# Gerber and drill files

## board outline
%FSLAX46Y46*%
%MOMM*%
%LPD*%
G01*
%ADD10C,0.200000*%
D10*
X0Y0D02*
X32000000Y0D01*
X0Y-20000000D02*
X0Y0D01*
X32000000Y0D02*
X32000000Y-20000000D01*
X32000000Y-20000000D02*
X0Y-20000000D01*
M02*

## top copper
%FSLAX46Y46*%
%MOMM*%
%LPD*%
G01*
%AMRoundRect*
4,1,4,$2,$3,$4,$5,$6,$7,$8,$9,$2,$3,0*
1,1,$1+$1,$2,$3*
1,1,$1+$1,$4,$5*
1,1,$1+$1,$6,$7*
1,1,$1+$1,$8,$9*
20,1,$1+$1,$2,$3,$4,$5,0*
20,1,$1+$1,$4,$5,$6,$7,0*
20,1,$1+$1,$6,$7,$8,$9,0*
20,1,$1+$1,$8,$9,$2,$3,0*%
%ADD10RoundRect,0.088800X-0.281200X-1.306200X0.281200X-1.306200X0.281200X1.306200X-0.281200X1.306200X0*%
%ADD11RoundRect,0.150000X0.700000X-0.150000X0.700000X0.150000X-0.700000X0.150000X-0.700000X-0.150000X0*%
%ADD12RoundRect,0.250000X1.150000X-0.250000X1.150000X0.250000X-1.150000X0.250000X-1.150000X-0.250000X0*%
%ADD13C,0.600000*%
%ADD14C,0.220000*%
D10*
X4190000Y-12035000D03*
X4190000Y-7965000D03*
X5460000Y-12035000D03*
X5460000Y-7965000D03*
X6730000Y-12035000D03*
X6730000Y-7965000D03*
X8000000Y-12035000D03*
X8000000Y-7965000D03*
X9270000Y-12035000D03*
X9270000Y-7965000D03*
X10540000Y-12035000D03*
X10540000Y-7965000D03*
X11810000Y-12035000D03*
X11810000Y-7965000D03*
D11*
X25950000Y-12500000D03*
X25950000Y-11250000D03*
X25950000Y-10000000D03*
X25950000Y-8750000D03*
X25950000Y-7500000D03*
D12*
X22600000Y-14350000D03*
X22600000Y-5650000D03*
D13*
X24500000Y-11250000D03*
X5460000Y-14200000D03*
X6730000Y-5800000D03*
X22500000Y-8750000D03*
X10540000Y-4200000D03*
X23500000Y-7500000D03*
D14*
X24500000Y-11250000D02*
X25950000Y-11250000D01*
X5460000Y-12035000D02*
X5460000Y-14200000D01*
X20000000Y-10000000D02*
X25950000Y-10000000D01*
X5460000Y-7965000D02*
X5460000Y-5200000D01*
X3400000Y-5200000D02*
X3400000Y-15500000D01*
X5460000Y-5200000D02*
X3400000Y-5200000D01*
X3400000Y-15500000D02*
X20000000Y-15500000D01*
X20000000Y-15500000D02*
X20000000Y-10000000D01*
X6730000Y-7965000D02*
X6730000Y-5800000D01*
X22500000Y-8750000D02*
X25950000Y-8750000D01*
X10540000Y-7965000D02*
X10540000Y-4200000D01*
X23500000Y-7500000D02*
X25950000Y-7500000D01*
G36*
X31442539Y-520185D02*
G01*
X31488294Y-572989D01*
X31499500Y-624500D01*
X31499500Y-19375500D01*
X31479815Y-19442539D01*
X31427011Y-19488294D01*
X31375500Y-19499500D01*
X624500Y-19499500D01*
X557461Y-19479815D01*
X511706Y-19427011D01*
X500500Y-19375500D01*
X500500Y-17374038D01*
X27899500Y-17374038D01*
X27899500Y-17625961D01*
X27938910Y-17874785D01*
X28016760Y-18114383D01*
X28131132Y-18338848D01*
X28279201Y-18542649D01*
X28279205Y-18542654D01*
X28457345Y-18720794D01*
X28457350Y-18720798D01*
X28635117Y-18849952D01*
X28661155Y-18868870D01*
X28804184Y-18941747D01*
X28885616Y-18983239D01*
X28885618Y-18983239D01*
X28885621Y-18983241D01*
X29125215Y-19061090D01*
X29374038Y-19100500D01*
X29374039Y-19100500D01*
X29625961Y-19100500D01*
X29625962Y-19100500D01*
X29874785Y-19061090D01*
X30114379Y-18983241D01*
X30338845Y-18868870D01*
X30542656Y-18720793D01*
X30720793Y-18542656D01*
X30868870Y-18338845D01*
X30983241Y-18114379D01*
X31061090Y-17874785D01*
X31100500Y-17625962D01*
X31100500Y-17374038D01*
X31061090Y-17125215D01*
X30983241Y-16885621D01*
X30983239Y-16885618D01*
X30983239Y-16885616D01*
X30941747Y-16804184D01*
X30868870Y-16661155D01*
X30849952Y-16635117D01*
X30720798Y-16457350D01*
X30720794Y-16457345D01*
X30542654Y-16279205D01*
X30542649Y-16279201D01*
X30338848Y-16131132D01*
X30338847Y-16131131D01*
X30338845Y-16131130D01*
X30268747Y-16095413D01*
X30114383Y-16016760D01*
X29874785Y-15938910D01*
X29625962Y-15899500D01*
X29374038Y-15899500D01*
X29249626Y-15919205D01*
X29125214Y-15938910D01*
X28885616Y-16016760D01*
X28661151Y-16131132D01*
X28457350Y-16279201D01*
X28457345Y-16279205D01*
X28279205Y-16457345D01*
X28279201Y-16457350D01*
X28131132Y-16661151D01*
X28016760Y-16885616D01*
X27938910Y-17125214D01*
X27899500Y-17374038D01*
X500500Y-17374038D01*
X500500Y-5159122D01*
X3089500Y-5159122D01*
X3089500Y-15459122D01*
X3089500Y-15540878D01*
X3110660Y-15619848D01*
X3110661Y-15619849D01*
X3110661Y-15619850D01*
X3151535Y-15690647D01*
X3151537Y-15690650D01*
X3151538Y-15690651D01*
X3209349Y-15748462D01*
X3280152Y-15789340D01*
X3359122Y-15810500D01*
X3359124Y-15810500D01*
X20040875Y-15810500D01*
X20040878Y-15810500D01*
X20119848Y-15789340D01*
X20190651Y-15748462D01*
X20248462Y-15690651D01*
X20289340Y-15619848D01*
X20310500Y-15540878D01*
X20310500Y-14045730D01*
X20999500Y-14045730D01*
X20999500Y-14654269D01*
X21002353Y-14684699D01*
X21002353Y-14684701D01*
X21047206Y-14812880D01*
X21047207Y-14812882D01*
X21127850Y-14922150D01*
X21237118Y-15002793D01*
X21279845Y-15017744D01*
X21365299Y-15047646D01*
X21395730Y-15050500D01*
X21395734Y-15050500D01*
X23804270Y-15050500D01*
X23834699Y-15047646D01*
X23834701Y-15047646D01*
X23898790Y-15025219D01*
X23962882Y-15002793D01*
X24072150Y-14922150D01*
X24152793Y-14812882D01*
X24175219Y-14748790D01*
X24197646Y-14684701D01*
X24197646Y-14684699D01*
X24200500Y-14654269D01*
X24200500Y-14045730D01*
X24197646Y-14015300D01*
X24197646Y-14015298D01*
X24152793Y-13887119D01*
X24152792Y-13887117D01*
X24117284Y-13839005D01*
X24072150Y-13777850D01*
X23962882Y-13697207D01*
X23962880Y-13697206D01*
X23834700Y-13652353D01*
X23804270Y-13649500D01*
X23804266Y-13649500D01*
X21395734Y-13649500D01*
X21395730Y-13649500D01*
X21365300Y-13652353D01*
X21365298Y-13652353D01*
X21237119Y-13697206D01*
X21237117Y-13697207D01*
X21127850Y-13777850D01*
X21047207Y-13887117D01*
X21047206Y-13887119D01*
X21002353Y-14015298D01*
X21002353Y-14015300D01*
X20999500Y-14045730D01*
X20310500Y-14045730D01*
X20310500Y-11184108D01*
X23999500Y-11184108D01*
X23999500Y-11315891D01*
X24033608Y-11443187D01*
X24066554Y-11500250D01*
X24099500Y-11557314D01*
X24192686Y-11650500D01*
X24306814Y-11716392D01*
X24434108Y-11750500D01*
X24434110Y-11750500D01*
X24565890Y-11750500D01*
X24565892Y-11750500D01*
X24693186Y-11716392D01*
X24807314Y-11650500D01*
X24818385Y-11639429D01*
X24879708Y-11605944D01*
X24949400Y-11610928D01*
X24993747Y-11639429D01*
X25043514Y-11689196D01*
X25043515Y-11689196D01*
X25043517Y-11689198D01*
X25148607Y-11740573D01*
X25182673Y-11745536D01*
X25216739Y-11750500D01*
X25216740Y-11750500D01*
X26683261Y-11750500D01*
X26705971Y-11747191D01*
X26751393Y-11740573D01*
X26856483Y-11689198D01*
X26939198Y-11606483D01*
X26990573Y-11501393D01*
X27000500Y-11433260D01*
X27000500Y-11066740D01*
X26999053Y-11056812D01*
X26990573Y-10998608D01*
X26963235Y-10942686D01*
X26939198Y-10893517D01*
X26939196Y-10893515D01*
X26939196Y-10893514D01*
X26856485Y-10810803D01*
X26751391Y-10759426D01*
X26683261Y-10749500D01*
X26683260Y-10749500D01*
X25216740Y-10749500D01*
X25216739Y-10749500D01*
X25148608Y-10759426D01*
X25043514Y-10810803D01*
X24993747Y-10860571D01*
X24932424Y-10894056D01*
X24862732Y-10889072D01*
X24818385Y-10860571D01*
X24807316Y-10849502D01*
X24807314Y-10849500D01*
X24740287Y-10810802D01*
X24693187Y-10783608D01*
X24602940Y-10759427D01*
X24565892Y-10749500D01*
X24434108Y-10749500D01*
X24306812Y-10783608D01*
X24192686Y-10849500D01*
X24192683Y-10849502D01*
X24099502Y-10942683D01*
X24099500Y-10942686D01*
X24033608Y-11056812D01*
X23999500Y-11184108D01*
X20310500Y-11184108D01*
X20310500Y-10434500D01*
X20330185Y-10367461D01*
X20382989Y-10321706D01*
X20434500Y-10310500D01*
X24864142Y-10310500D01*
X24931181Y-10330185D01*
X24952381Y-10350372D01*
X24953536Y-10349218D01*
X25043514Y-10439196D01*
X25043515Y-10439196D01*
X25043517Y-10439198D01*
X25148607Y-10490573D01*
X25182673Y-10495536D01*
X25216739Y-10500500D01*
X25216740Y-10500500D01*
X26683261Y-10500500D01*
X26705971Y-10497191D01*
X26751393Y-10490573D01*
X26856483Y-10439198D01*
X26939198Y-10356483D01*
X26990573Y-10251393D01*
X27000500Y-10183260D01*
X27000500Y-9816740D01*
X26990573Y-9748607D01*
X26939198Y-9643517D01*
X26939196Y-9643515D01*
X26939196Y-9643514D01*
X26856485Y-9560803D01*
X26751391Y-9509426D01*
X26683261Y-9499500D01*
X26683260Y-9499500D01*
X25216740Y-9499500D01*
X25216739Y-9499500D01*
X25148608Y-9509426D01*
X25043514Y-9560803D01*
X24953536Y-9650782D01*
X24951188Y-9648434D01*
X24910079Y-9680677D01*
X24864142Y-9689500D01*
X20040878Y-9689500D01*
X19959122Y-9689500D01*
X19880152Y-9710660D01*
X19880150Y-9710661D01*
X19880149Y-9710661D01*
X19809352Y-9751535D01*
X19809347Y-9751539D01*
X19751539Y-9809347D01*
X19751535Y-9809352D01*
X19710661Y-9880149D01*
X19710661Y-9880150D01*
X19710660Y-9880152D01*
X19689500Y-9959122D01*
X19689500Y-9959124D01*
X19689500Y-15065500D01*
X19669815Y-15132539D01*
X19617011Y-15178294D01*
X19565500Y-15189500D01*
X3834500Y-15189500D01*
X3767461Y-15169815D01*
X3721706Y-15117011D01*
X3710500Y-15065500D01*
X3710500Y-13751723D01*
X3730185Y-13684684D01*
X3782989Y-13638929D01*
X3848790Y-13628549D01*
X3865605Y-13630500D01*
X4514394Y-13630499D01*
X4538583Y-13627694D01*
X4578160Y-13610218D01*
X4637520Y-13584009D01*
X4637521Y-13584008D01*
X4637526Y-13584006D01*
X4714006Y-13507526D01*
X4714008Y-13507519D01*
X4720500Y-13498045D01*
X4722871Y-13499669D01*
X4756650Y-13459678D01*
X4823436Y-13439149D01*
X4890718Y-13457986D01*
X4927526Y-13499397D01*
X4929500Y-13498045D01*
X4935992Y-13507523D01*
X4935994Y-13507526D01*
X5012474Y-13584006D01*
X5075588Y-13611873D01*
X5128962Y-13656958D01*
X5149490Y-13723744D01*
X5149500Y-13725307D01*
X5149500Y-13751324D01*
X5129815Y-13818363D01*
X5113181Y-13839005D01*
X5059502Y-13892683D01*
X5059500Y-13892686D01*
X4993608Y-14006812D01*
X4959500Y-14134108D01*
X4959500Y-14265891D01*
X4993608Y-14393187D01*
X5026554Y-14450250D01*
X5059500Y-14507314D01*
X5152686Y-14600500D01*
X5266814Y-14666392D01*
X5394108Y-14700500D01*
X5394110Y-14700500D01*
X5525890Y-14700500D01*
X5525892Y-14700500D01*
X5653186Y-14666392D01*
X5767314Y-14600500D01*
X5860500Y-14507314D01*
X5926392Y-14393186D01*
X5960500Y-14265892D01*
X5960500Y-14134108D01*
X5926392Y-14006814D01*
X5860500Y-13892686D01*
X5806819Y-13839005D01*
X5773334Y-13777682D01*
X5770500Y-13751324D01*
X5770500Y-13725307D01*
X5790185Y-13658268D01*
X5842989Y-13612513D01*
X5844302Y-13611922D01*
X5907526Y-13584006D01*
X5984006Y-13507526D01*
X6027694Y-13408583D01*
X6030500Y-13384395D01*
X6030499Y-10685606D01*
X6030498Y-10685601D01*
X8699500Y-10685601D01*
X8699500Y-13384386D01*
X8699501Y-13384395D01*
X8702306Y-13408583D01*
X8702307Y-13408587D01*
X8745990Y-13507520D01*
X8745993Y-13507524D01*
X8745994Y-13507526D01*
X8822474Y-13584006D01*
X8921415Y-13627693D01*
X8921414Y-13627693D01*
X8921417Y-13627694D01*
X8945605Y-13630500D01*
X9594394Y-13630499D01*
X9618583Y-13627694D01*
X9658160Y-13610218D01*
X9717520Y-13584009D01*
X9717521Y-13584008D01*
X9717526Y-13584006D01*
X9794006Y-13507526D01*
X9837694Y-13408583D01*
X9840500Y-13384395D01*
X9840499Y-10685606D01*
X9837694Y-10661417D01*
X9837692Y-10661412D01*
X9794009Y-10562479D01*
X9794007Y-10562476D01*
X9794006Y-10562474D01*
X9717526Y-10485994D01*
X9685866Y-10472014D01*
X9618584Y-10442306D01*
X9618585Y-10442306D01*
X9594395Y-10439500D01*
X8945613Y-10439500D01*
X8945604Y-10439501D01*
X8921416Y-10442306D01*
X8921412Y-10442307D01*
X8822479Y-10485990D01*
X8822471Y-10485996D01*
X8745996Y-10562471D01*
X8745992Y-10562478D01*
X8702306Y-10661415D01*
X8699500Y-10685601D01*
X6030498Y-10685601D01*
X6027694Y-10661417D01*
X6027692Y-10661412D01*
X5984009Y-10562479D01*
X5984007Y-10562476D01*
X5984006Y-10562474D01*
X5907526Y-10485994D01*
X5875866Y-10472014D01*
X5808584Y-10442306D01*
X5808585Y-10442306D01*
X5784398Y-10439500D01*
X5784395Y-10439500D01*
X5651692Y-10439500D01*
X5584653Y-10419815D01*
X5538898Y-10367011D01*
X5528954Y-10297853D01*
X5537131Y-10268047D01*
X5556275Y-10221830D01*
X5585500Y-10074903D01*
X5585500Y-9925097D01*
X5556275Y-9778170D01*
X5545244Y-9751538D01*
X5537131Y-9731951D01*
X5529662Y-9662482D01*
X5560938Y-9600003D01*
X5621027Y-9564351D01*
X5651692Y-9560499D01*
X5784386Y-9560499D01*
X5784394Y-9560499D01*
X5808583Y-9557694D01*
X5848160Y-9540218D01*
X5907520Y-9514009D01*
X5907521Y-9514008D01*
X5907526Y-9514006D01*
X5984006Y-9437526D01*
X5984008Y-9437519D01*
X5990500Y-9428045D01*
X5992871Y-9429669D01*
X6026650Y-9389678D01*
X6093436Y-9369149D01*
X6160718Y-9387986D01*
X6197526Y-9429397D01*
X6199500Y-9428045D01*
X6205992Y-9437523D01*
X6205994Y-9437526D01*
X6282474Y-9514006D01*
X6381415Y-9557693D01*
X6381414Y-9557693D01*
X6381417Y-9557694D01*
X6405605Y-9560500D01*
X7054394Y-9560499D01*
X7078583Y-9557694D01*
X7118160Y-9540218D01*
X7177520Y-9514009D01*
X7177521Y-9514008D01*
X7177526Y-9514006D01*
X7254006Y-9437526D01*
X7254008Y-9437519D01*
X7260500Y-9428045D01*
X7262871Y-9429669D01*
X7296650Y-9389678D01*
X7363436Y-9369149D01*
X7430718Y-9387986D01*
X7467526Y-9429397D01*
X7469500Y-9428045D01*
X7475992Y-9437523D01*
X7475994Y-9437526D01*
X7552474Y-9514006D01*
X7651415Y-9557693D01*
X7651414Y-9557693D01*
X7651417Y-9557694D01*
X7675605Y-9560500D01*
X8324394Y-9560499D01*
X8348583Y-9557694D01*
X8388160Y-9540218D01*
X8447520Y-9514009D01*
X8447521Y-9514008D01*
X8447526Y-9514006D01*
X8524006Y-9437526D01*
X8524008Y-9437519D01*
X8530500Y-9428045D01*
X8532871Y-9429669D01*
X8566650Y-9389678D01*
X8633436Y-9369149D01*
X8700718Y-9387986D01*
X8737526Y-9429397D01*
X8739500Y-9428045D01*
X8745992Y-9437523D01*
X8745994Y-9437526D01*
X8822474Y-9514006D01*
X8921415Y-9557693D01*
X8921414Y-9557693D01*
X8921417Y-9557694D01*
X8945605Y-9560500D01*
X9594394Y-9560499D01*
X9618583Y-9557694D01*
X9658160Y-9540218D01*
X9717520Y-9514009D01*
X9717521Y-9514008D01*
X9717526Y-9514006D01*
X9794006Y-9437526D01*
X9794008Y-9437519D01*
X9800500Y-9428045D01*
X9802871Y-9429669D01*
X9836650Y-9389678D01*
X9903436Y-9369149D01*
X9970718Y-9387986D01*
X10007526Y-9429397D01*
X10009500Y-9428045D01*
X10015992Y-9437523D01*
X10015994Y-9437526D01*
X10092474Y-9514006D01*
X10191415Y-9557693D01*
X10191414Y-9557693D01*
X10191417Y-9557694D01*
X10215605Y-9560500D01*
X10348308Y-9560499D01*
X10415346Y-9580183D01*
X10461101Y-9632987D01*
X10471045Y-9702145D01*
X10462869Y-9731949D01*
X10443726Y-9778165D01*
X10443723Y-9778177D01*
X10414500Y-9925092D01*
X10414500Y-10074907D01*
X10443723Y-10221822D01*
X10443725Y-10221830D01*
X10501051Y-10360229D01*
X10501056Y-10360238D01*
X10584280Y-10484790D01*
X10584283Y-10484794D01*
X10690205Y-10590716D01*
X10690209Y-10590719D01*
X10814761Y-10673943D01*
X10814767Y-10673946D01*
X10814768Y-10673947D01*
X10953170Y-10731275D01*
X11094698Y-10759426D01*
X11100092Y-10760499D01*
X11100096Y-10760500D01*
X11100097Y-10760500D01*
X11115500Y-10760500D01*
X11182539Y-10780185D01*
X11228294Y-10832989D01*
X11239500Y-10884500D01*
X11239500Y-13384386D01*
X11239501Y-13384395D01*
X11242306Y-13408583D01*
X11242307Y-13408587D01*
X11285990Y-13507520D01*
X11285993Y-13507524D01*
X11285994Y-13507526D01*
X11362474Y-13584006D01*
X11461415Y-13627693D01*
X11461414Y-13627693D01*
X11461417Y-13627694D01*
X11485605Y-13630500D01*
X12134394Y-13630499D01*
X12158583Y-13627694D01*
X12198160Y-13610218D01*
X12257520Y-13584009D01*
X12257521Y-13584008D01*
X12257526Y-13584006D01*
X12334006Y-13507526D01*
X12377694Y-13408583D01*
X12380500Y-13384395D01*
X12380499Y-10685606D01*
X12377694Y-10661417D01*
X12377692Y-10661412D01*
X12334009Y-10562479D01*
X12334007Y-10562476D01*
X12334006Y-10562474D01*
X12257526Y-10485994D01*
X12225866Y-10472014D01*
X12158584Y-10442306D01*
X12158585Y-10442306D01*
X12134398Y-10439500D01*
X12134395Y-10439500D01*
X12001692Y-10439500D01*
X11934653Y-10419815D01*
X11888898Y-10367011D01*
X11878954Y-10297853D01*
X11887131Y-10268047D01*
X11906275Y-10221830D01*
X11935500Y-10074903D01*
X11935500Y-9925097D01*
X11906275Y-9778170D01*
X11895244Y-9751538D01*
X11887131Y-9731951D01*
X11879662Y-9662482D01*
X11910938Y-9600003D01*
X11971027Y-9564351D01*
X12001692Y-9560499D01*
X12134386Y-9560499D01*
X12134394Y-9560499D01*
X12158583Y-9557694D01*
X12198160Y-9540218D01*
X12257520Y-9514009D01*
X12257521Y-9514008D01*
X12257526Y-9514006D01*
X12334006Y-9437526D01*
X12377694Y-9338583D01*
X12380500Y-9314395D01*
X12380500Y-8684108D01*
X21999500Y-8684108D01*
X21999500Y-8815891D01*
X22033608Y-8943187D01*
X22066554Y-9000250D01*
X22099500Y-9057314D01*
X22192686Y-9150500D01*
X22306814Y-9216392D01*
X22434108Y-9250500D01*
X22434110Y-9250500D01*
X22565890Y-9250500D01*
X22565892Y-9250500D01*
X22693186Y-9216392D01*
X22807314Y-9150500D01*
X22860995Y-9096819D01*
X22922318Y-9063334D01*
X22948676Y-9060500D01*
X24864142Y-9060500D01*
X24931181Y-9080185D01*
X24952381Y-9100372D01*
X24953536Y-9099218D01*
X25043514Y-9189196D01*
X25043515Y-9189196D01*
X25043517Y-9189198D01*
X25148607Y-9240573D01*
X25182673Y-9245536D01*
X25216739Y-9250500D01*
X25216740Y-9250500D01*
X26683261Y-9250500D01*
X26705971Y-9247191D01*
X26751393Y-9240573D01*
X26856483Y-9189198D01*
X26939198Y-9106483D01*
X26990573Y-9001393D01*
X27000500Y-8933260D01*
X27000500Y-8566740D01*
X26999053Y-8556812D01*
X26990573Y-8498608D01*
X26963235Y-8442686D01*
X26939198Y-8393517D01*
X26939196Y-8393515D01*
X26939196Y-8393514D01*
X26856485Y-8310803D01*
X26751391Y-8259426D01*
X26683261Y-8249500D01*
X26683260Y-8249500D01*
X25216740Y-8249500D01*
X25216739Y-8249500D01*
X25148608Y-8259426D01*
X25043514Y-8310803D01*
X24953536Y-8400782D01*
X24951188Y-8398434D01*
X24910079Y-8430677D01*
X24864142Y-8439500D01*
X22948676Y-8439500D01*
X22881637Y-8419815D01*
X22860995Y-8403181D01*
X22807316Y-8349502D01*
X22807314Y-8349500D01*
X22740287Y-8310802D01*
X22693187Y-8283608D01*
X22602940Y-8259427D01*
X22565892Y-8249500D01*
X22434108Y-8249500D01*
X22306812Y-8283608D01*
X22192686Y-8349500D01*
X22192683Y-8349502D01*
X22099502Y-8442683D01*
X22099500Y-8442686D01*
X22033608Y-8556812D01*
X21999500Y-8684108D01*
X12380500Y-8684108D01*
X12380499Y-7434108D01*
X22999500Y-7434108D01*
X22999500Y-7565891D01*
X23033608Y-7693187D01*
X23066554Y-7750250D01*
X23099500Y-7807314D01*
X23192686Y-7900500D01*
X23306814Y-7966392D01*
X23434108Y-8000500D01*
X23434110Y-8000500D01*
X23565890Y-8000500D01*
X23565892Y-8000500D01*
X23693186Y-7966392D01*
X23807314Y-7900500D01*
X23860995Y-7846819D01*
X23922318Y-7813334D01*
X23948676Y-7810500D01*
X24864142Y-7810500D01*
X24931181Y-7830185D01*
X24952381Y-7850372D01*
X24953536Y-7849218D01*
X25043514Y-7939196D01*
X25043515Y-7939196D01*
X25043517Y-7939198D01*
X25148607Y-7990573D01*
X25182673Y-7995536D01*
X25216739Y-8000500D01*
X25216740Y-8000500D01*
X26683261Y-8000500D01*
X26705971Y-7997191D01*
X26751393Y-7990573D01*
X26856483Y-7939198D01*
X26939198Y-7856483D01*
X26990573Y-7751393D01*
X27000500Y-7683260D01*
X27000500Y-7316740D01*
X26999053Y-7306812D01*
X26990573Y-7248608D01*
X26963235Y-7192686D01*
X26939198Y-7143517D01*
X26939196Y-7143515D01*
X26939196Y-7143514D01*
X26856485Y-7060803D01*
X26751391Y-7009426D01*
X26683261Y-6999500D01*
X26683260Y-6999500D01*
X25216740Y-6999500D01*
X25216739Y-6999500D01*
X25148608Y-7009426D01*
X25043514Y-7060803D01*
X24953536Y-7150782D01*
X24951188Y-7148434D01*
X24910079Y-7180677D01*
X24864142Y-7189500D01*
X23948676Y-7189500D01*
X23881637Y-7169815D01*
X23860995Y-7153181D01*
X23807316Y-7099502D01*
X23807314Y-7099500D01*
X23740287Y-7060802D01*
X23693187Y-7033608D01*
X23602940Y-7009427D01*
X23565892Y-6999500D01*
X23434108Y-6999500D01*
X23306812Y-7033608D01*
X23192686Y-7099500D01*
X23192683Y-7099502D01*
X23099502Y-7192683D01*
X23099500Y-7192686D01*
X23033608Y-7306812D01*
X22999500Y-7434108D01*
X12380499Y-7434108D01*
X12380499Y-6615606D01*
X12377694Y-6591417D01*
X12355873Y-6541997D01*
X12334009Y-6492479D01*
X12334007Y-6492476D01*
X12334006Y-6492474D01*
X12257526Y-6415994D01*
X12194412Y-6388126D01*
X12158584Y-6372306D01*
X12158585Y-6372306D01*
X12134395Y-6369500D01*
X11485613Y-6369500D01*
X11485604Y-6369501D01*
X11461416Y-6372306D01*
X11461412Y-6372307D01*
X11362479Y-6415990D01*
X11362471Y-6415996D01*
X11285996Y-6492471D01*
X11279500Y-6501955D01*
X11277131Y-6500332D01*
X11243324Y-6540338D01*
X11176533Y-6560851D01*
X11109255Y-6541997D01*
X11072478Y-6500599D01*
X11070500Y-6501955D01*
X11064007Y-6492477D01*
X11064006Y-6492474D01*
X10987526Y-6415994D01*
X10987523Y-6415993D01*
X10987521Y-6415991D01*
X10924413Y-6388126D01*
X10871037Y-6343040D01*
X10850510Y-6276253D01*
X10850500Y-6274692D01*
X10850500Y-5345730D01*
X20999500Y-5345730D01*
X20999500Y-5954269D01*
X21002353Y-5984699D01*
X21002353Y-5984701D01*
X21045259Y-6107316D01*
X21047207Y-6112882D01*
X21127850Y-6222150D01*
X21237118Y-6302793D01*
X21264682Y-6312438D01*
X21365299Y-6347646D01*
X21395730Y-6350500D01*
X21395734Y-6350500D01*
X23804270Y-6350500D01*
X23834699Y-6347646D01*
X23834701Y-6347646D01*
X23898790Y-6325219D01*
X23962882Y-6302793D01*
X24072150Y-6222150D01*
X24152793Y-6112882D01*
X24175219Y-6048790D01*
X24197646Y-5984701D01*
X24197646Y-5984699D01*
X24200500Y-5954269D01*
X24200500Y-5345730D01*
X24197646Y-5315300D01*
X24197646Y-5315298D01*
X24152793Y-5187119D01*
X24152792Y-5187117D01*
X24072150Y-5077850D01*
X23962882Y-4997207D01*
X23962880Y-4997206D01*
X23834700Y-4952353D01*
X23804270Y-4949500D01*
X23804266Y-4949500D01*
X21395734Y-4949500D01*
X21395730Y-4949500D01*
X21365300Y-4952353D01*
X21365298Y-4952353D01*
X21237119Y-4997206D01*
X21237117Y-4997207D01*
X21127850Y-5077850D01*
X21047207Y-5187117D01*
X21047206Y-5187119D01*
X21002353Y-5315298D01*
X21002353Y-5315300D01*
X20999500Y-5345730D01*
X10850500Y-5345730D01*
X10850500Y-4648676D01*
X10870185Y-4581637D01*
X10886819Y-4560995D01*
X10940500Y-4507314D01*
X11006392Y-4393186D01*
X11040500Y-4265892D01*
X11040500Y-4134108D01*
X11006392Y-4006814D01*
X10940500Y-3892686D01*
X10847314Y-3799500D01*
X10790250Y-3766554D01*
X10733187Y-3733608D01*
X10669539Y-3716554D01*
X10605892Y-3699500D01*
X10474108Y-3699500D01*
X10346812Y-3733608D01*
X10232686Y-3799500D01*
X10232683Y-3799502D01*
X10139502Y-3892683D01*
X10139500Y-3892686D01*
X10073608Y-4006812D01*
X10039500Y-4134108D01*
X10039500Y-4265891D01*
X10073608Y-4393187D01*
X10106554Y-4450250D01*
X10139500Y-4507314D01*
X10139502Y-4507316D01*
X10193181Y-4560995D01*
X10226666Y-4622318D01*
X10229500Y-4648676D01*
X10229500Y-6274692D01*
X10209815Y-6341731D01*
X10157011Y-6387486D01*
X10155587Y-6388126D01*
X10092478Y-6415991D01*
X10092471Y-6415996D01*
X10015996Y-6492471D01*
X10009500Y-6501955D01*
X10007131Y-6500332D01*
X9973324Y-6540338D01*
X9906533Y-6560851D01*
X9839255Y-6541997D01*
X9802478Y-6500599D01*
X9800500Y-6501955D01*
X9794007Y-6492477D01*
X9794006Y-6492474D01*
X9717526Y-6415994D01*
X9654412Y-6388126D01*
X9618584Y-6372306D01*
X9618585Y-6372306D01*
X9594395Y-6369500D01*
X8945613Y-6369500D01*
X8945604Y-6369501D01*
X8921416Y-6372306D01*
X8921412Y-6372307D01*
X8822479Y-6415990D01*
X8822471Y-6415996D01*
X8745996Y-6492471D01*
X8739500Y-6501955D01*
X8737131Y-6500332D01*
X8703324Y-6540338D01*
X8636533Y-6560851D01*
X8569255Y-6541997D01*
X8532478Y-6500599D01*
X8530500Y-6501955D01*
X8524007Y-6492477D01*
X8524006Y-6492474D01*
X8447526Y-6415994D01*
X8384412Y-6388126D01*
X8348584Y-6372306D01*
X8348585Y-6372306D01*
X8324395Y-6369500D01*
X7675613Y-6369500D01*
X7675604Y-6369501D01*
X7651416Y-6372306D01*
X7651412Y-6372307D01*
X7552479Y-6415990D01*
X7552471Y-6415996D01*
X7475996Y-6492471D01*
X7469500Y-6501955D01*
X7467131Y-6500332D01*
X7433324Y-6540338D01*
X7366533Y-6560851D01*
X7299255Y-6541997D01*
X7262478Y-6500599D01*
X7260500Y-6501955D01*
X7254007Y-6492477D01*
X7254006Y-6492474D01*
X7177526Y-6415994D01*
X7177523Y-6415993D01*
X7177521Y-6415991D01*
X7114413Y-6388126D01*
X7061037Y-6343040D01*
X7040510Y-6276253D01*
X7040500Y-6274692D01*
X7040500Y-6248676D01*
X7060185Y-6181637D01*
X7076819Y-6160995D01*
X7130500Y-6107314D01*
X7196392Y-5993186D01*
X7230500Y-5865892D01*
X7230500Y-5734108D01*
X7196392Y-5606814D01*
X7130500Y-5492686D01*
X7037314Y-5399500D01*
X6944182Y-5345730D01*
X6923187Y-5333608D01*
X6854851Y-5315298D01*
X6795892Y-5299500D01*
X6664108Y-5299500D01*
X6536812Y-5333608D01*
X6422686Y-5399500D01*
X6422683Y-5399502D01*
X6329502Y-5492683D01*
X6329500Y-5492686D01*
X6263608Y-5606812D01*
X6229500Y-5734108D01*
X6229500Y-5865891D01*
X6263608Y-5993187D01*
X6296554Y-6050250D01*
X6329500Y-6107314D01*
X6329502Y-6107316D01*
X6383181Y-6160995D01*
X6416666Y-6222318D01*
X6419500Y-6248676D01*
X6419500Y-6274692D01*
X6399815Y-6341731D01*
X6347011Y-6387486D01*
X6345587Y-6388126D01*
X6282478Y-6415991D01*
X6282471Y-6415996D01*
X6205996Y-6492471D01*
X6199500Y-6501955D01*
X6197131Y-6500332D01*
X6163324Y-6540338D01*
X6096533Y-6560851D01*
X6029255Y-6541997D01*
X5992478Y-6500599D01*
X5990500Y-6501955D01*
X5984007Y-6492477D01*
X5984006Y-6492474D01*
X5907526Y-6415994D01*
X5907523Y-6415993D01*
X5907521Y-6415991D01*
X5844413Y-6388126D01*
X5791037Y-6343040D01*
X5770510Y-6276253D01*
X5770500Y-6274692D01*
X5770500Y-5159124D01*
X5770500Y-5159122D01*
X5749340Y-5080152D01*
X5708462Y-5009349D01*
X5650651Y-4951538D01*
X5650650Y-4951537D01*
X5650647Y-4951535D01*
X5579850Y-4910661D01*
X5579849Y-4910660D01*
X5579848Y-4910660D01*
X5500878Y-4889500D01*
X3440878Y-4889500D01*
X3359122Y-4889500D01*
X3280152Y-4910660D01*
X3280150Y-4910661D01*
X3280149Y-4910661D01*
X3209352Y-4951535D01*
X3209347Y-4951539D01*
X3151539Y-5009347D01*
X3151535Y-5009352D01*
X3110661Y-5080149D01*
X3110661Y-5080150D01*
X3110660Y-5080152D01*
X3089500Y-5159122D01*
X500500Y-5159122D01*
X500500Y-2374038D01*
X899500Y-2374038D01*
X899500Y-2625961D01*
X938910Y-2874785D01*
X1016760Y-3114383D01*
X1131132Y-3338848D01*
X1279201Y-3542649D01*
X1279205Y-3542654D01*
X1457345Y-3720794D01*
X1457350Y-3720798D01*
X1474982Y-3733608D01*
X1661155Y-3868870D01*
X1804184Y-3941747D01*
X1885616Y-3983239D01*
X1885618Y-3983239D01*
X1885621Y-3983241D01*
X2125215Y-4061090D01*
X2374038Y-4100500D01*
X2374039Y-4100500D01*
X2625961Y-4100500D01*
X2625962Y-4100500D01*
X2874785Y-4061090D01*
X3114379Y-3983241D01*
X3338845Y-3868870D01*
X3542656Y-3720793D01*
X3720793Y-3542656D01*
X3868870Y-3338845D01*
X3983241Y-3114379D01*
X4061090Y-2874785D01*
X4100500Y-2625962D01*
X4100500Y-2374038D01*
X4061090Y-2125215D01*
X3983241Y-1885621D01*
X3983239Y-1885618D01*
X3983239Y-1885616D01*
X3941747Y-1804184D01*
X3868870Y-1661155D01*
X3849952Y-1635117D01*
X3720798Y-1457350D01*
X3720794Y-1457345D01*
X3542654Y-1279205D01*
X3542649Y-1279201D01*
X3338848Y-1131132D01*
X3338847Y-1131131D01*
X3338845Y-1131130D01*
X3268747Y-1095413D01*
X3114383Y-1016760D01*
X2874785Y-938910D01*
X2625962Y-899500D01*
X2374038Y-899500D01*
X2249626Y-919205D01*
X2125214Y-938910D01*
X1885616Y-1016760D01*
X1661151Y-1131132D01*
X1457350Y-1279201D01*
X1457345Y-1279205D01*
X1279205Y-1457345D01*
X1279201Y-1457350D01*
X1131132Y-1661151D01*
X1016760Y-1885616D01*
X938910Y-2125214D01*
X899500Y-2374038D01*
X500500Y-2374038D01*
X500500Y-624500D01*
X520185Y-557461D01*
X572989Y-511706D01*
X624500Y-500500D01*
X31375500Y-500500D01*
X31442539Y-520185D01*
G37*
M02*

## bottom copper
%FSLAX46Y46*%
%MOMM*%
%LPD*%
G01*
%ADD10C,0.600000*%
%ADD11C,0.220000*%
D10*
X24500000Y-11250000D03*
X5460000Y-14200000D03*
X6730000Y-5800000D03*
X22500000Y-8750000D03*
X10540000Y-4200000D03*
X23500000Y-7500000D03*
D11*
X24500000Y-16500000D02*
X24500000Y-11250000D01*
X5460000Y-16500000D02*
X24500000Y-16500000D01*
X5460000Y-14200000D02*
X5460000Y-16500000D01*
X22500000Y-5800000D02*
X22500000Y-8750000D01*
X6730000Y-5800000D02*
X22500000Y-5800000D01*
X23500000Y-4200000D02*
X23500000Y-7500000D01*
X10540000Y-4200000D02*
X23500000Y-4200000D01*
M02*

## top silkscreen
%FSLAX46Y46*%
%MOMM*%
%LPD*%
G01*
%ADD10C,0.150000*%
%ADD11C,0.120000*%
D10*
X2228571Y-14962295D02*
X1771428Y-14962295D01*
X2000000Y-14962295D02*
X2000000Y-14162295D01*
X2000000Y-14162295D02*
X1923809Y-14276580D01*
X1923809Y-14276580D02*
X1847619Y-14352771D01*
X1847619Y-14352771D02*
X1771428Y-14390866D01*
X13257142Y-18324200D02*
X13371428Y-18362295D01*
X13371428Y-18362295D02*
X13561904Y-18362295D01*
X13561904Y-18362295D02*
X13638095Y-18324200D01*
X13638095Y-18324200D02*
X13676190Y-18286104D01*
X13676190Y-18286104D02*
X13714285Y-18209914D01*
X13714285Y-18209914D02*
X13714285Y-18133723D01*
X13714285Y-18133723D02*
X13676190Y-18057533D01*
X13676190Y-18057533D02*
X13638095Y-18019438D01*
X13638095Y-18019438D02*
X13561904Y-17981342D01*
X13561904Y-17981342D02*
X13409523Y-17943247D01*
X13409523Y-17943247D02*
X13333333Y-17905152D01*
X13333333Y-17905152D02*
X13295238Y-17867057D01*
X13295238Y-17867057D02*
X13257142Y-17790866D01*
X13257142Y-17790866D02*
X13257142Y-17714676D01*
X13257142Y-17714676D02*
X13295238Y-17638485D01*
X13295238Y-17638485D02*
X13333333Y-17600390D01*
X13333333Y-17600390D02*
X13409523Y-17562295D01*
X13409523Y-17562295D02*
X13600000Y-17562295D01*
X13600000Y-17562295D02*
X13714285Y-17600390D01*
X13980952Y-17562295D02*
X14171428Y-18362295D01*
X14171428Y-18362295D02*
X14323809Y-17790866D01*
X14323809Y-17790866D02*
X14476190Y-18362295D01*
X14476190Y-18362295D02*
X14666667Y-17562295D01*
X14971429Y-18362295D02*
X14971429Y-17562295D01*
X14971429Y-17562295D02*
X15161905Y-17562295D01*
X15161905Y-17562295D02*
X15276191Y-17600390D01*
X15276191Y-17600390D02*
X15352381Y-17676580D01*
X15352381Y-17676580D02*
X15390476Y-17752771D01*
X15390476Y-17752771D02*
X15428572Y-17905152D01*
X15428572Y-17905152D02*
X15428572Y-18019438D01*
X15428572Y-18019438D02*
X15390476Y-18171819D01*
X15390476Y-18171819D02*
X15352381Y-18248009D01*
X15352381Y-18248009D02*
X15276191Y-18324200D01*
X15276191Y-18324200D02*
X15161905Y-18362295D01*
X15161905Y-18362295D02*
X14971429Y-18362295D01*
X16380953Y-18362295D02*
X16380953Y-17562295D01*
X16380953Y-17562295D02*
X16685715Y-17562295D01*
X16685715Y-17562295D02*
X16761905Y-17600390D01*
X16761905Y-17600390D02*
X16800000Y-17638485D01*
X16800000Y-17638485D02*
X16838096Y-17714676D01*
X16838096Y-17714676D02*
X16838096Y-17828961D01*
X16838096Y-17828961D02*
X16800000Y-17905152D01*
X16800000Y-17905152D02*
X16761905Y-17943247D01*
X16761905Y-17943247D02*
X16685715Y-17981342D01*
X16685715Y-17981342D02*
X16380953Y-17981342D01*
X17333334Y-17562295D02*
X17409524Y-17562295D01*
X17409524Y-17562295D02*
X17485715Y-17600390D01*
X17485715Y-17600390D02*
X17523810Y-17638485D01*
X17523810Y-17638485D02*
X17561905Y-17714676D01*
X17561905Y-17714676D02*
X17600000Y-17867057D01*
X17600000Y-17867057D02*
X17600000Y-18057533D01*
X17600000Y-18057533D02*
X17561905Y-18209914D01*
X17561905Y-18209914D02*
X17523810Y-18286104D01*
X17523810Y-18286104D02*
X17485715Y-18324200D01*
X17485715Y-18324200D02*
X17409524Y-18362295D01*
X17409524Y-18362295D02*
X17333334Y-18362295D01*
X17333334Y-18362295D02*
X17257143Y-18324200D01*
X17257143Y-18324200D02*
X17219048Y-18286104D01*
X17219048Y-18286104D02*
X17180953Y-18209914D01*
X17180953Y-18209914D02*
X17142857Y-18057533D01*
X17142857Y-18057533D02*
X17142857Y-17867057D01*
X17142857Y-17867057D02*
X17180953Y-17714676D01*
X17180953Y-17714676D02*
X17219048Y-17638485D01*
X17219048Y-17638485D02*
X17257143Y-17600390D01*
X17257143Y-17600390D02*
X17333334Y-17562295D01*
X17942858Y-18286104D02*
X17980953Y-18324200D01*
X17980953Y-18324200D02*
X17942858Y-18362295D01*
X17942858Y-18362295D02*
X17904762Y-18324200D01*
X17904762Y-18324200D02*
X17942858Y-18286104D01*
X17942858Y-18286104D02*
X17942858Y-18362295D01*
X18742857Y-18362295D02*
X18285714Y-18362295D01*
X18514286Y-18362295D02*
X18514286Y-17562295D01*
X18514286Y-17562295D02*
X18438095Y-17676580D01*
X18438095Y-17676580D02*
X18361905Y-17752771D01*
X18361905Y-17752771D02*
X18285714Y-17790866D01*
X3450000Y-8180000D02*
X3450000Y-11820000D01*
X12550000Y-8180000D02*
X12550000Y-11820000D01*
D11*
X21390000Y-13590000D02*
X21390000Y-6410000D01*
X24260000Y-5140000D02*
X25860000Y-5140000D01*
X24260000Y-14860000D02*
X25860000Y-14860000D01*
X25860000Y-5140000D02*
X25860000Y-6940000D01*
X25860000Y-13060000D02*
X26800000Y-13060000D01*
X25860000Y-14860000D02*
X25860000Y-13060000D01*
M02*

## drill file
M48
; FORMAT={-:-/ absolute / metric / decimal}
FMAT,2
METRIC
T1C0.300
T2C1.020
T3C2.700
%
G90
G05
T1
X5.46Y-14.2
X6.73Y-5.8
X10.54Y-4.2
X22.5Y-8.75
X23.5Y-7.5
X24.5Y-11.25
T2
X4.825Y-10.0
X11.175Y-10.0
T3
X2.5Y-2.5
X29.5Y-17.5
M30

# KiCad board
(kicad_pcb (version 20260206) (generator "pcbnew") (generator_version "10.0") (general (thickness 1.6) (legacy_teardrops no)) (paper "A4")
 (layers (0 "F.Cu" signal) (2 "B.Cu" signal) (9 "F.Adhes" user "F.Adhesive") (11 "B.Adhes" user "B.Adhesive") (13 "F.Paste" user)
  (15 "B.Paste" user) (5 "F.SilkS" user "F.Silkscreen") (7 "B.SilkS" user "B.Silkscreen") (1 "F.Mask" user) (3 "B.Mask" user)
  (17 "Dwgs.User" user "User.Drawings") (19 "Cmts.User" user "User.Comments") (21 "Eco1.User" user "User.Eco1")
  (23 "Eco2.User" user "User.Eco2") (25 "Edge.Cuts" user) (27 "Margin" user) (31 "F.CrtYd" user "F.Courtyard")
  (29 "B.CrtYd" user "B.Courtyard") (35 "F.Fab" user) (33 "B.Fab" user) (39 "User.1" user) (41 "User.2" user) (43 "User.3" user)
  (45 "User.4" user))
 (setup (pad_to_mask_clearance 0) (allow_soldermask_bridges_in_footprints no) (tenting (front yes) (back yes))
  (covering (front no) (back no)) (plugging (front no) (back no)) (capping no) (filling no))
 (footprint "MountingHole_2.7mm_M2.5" (layer "F.Cu") (at 2.5 2.5)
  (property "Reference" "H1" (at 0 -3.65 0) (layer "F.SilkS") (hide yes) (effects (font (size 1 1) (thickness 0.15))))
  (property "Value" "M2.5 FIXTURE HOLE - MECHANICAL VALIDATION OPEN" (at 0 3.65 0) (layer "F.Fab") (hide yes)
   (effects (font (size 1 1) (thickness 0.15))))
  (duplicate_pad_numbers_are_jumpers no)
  (pad "" np_thru_hole circle (at 0 0) (size 2.7 2.7) (drill 2.7) (layers "*.Cu" "*.Mask")))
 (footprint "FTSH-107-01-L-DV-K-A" (layer "F.Cu") (at 8 10)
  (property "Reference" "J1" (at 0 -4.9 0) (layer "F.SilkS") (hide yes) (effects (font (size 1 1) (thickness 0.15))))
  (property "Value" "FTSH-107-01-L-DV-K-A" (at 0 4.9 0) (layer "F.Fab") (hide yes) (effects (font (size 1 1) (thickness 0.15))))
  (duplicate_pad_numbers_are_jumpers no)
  (fp_line (start -4.55 -1.82) (end -4.55 1.82) (stroke (width 0.15) (type solid)) (layer "F.SilkS"))
  (fp_line (start 4.55 -1.82) (end 4.55 1.82) (stroke (width 0.15) (type solid)) (layer "F.SilkS"))
  (pad "" np_thru_hole circle (at -3.175 0) (size 1.02 1.02) (drill 1.02) (layers "*.Cu" "*.Mask"))
  (pad "" np_thru_hole circle (at 3.175 0) (size 1.02 1.02) (drill 1.02) (layers "*.Cu" "*.Mask"))
  (pad "1" smd roundrect (at -3.81 2.035) (size 0.74 2.79) (layers "F.Cu" "F.Mask" "F.Paste") (roundrect_rratio 0.12))
  (pad "2" smd roundrect (at -3.81 -2.035) (size 0.74 2.79) (layers "F.Cu" "F.Mask" "F.Paste") (roundrect_rratio 0.12))
  (pad "3" smd roundrect (at -2.54 2.035) (size 0.74 2.79) (layers "F.Cu" "F.Mask" "F.Paste") (roundrect_rratio 0.12) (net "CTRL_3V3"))
  (pad "4" smd roundrect (at -2.54 -2.035) (size 0.74 2.79) (layers "F.Cu" "F.Mask" "F.Paste") (roundrect_rratio 0.12) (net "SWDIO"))
  (pad "5" smd roundrect (at -1.27 2.035) (size 0.74 2.79) (layers "F.Cu" "F.Mask" "F.Paste") (roundrect_rratio 0.12) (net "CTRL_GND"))
  (pad "6" smd roundrect (at -1.27 -2.035) (size 0.74 2.79) (layers "F.Cu" "F.Mask" "F.Paste") (roundrect_rratio 0.12) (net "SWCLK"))
  (pad "7" smd roundrect (at 0 2.035) (size 0.74 2.79) (layers "F.Cu" "F.Mask" "F.Paste") (roundrect_rratio 0.12) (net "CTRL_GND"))
  (pad "8" smd roundrect (at 0 -2.035) (size 0.74 2.79) (layers "F.Cu" "F.Mask" "F.Paste") (roundrect_rratio 0.12))
  (pad "9" smd roundrect (at 1.27 2.035) (size 0.74 2.79) (layers "F.Cu" "F.Mask" "F.Paste") (roundrect_rratio 0.12))
  (pad "10" smd roundrect (at 1.27 -2.035) (size 0.74 2.79) (layers "F.Cu" "F.Mask" "F.Paste") (roundrect_rratio 0.12))
  (pad "11" smd roundrect (at 2.54 2.035) (size 0.74 2.79) (layers "F.Cu" "F.Mask" "F.Paste") (roundrect_rratio 0.12) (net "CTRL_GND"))
  (pad "12" smd roundrect (at 2.54 -2.035) (size 0.74 2.79) (layers "F.Cu" "F.Mask" "F.Paste") (roundrect_rratio 0.12) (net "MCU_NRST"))
  (pad "13" smd roundrect (at 3.81 2.035) (size 0.74 2.79) (layers "F.Cu" "F.Mask" "F.Paste") (roundrect_rratio 0.12))
  (pad "14" smd roundrect (at 3.81 -2.035) (size 0.74 2.79) (layers "F.Cu" "F.Mask" "F.Paste") (roundrect_rratio 0.12)))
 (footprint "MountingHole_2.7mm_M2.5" (layer "F.Cu") (at 29.5 17.5)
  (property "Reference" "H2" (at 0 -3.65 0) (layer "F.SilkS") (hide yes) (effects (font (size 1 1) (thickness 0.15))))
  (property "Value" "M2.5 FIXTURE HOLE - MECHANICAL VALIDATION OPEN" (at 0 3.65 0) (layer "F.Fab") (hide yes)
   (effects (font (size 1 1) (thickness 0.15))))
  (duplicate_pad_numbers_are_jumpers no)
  (pad "" np_thru_hole circle (at 0 0) (size 2.7 2.7) (drill 2.7) (layers "*.Cu" "*.Mask")))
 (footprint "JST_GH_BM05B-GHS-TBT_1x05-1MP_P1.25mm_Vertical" (layer "F.Cu") (at 24 10 90)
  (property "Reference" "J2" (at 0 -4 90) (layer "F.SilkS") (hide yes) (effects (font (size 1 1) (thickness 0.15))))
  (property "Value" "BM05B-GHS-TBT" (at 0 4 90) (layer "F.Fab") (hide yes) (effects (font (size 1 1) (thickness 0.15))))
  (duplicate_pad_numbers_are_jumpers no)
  (fp_line (start -3.59 -2.61) (end 3.59 -2.61) (stroke (width 0.12) (type solid)) (layer "F.SilkS"))
  (fp_line (start 4.86 0.26) (end 4.86 1.86) (stroke (width 0.12) (type solid)) (layer "F.SilkS"))
  (fp_line (start -4.86 0.26) (end -4.86 1.86) (stroke (width 0.12) (type solid)) (layer "F.SilkS"))
  (fp_line (start 4.86 1.86) (end 3.06 1.86) (stroke (width 0.12) (type solid)) (layer "F.SilkS"))
  (fp_line (start -3.06 1.86) (end -3.06 2.8) (stroke (width 0.12) (type solid)) (layer "F.SilkS"))
  (fp_line (start -4.86 1.86) (end -3.06 1.86) (stroke (width 0.12) (type solid)) (layer "F.SilkS"))
  (pad "1" smd roundrect (at -2.5 1.95 90) (size 0.6 1.7) (layers "F.Cu" "F.Mask" "F.Paste") (roundrect_rratio 0.25) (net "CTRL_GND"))
  (pad "2" smd roundrect (at -1.25 1.95 90) (size 0.6 1.7) (layers "F.Cu" "F.Mask" "F.Paste") (roundrect_rratio 0.25) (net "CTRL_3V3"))
  (pad "3" smd roundrect (at 0 1.95 90) (size 0.6 1.7) (layers "F.Cu" "F.Mask" "F.Paste") (roundrect_rratio 0.25) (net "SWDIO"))
  (pad "4" smd roundrect (at 1.25 1.95 90) (size 0.6 1.7) (layers "F.Cu" "F.Mask" "F.Paste") (roundrect_rratio 0.25) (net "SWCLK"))
  (pad "5" smd roundrect (at 2.5 1.95 90) (size 0.6 1.7) (layers "F.Cu" "F.Mask" "F.Paste") (roundrect_rratio 0.25) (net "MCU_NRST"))
  (pad "MP" smd roundrect (at -4.35 -1.4 90) (size 1 2.8) (layers "F.Cu" "F.Mask" "F.Paste") (roundrect_rratio 0.25))
  (pad "MP" smd roundrect (at 4.35 -1.4 90) (size 1 2.8) (layers "F.Cu" "F.Mask" "F.Paste") (roundrect_rratio 0.25)))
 (gr_line (start 0 0) (end 32 0) (stroke (width 0.2) (type default)) (layer "Edge.Cuts"))
 (gr_line (start 0 20) (end 0 0) (stroke (width 0.2) (type default)) (layer "Edge.Cuts"))
 (gr_line (start 32 0) (end 32 20) (stroke (width 0.2) (type default)) (layer "Edge.Cuts"))
 (gr_line (start 32 20) (end 0 20) (stroke (width 0.2) (type default)) (layer "Edge.Cuts"))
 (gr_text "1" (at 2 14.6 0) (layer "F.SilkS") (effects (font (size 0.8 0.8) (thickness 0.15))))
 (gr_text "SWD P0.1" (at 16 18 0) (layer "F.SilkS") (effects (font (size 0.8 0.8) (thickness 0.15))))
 (segment (start 24.5 11.25) (end 25.95 11.25) (width 0.22) (layer "F.Cu") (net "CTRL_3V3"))
 (segment (start 5.46 12.035) (end 5.46 14.2) (width 0.22) (layer "F.Cu") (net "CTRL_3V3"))
 (via (at 24.5 11.25) (size 0.6) (drill 0.3) (layers "F.Cu" "B.Cu") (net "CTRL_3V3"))
 (via (at 5.46 14.2) (size 0.6) (drill 0.3) (layers "F.Cu" "B.Cu") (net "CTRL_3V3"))
 (segment (start 24.5 16.5) (end 24.5 11.25) (width 0.22) (layer "B.Cu") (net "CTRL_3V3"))
 (segment (start 5.46 16.5) (end 24.5 16.5) (width 0.22) (layer "B.Cu") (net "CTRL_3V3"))
 (segment (start 5.46 14.2) (end 5.46 16.5) (width 0.22) (layer "B.Cu") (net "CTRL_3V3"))
 (segment (start 20 10) (end 25.95 10) (width 0.22) (layer "F.Cu") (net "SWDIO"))
 (segment (start 5.46 7.965) (end 5.46 5.2) (width 0.22) (layer "F.Cu") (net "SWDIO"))
 (segment (start 3.4 5.2) (end 3.4 15.5) (width 0.22) (layer "F.Cu") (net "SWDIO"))
 (segment (start 5.46 5.2) (end 3.4 5.2) (width 0.22) (layer "F.Cu") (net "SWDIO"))
 (segment (start 3.4 15.5) (end 20 15.5) (width 0.22) (layer "F.Cu") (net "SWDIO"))
 (segment (start 20 15.5) (end 20 10) (width 0.22) (layer "F.Cu") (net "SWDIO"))
 (segment (start 6.73 7.965) (end 6.73 5.8) (width 0.22) (layer "F.Cu") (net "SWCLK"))
 (segment (start 22.5 8.75) (end 25.95 8.75) (width 0.22) (layer "F.Cu") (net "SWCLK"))
 (via (at 6.73 5.8) (size 0.6) (drill 0.3) (layers "F.Cu" "B.Cu") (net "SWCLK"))
 (via (at 22.5 8.75) (size 0.6) (drill 0.3) (layers "F.Cu" "B.Cu") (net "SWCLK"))
 (segment (start 22.5 5.8) (end 22.5 8.75) (width 0.22) (layer "B.Cu") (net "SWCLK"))
 (segment (start 6.73 5.8) (end 22.5 5.8) (width 0.22) (layer "B.Cu") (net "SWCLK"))
 (segment (start 10.54 7.965) (end 10.54 4.2) (width 0.22) (layer "F.Cu") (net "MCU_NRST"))
 (segment (start 23.5 7.5) (end 25.95 7.5) (width 0.22) (layer "F.Cu") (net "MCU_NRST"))
 (via (at 10.54 4.2) (size 0.6) (drill 0.3) (layers "F.Cu" "B.Cu") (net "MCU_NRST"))
 (via (at 23.5 7.5) (size 0.6) (drill 0.3) (layers "F.Cu" "B.Cu") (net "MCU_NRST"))
 (segment (start 23.5 4.2) (end 23.5 7.5) (width 0.22) (layer "B.Cu") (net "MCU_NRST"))
 (segment (start 10.54 4.2) (end 23.5 4.2) (width 0.22) (layer "B.Cu") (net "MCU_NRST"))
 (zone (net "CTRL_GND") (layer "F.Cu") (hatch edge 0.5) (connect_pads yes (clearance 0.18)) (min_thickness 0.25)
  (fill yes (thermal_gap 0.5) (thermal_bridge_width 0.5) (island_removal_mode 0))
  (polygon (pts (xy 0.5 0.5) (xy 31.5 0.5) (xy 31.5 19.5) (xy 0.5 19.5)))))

